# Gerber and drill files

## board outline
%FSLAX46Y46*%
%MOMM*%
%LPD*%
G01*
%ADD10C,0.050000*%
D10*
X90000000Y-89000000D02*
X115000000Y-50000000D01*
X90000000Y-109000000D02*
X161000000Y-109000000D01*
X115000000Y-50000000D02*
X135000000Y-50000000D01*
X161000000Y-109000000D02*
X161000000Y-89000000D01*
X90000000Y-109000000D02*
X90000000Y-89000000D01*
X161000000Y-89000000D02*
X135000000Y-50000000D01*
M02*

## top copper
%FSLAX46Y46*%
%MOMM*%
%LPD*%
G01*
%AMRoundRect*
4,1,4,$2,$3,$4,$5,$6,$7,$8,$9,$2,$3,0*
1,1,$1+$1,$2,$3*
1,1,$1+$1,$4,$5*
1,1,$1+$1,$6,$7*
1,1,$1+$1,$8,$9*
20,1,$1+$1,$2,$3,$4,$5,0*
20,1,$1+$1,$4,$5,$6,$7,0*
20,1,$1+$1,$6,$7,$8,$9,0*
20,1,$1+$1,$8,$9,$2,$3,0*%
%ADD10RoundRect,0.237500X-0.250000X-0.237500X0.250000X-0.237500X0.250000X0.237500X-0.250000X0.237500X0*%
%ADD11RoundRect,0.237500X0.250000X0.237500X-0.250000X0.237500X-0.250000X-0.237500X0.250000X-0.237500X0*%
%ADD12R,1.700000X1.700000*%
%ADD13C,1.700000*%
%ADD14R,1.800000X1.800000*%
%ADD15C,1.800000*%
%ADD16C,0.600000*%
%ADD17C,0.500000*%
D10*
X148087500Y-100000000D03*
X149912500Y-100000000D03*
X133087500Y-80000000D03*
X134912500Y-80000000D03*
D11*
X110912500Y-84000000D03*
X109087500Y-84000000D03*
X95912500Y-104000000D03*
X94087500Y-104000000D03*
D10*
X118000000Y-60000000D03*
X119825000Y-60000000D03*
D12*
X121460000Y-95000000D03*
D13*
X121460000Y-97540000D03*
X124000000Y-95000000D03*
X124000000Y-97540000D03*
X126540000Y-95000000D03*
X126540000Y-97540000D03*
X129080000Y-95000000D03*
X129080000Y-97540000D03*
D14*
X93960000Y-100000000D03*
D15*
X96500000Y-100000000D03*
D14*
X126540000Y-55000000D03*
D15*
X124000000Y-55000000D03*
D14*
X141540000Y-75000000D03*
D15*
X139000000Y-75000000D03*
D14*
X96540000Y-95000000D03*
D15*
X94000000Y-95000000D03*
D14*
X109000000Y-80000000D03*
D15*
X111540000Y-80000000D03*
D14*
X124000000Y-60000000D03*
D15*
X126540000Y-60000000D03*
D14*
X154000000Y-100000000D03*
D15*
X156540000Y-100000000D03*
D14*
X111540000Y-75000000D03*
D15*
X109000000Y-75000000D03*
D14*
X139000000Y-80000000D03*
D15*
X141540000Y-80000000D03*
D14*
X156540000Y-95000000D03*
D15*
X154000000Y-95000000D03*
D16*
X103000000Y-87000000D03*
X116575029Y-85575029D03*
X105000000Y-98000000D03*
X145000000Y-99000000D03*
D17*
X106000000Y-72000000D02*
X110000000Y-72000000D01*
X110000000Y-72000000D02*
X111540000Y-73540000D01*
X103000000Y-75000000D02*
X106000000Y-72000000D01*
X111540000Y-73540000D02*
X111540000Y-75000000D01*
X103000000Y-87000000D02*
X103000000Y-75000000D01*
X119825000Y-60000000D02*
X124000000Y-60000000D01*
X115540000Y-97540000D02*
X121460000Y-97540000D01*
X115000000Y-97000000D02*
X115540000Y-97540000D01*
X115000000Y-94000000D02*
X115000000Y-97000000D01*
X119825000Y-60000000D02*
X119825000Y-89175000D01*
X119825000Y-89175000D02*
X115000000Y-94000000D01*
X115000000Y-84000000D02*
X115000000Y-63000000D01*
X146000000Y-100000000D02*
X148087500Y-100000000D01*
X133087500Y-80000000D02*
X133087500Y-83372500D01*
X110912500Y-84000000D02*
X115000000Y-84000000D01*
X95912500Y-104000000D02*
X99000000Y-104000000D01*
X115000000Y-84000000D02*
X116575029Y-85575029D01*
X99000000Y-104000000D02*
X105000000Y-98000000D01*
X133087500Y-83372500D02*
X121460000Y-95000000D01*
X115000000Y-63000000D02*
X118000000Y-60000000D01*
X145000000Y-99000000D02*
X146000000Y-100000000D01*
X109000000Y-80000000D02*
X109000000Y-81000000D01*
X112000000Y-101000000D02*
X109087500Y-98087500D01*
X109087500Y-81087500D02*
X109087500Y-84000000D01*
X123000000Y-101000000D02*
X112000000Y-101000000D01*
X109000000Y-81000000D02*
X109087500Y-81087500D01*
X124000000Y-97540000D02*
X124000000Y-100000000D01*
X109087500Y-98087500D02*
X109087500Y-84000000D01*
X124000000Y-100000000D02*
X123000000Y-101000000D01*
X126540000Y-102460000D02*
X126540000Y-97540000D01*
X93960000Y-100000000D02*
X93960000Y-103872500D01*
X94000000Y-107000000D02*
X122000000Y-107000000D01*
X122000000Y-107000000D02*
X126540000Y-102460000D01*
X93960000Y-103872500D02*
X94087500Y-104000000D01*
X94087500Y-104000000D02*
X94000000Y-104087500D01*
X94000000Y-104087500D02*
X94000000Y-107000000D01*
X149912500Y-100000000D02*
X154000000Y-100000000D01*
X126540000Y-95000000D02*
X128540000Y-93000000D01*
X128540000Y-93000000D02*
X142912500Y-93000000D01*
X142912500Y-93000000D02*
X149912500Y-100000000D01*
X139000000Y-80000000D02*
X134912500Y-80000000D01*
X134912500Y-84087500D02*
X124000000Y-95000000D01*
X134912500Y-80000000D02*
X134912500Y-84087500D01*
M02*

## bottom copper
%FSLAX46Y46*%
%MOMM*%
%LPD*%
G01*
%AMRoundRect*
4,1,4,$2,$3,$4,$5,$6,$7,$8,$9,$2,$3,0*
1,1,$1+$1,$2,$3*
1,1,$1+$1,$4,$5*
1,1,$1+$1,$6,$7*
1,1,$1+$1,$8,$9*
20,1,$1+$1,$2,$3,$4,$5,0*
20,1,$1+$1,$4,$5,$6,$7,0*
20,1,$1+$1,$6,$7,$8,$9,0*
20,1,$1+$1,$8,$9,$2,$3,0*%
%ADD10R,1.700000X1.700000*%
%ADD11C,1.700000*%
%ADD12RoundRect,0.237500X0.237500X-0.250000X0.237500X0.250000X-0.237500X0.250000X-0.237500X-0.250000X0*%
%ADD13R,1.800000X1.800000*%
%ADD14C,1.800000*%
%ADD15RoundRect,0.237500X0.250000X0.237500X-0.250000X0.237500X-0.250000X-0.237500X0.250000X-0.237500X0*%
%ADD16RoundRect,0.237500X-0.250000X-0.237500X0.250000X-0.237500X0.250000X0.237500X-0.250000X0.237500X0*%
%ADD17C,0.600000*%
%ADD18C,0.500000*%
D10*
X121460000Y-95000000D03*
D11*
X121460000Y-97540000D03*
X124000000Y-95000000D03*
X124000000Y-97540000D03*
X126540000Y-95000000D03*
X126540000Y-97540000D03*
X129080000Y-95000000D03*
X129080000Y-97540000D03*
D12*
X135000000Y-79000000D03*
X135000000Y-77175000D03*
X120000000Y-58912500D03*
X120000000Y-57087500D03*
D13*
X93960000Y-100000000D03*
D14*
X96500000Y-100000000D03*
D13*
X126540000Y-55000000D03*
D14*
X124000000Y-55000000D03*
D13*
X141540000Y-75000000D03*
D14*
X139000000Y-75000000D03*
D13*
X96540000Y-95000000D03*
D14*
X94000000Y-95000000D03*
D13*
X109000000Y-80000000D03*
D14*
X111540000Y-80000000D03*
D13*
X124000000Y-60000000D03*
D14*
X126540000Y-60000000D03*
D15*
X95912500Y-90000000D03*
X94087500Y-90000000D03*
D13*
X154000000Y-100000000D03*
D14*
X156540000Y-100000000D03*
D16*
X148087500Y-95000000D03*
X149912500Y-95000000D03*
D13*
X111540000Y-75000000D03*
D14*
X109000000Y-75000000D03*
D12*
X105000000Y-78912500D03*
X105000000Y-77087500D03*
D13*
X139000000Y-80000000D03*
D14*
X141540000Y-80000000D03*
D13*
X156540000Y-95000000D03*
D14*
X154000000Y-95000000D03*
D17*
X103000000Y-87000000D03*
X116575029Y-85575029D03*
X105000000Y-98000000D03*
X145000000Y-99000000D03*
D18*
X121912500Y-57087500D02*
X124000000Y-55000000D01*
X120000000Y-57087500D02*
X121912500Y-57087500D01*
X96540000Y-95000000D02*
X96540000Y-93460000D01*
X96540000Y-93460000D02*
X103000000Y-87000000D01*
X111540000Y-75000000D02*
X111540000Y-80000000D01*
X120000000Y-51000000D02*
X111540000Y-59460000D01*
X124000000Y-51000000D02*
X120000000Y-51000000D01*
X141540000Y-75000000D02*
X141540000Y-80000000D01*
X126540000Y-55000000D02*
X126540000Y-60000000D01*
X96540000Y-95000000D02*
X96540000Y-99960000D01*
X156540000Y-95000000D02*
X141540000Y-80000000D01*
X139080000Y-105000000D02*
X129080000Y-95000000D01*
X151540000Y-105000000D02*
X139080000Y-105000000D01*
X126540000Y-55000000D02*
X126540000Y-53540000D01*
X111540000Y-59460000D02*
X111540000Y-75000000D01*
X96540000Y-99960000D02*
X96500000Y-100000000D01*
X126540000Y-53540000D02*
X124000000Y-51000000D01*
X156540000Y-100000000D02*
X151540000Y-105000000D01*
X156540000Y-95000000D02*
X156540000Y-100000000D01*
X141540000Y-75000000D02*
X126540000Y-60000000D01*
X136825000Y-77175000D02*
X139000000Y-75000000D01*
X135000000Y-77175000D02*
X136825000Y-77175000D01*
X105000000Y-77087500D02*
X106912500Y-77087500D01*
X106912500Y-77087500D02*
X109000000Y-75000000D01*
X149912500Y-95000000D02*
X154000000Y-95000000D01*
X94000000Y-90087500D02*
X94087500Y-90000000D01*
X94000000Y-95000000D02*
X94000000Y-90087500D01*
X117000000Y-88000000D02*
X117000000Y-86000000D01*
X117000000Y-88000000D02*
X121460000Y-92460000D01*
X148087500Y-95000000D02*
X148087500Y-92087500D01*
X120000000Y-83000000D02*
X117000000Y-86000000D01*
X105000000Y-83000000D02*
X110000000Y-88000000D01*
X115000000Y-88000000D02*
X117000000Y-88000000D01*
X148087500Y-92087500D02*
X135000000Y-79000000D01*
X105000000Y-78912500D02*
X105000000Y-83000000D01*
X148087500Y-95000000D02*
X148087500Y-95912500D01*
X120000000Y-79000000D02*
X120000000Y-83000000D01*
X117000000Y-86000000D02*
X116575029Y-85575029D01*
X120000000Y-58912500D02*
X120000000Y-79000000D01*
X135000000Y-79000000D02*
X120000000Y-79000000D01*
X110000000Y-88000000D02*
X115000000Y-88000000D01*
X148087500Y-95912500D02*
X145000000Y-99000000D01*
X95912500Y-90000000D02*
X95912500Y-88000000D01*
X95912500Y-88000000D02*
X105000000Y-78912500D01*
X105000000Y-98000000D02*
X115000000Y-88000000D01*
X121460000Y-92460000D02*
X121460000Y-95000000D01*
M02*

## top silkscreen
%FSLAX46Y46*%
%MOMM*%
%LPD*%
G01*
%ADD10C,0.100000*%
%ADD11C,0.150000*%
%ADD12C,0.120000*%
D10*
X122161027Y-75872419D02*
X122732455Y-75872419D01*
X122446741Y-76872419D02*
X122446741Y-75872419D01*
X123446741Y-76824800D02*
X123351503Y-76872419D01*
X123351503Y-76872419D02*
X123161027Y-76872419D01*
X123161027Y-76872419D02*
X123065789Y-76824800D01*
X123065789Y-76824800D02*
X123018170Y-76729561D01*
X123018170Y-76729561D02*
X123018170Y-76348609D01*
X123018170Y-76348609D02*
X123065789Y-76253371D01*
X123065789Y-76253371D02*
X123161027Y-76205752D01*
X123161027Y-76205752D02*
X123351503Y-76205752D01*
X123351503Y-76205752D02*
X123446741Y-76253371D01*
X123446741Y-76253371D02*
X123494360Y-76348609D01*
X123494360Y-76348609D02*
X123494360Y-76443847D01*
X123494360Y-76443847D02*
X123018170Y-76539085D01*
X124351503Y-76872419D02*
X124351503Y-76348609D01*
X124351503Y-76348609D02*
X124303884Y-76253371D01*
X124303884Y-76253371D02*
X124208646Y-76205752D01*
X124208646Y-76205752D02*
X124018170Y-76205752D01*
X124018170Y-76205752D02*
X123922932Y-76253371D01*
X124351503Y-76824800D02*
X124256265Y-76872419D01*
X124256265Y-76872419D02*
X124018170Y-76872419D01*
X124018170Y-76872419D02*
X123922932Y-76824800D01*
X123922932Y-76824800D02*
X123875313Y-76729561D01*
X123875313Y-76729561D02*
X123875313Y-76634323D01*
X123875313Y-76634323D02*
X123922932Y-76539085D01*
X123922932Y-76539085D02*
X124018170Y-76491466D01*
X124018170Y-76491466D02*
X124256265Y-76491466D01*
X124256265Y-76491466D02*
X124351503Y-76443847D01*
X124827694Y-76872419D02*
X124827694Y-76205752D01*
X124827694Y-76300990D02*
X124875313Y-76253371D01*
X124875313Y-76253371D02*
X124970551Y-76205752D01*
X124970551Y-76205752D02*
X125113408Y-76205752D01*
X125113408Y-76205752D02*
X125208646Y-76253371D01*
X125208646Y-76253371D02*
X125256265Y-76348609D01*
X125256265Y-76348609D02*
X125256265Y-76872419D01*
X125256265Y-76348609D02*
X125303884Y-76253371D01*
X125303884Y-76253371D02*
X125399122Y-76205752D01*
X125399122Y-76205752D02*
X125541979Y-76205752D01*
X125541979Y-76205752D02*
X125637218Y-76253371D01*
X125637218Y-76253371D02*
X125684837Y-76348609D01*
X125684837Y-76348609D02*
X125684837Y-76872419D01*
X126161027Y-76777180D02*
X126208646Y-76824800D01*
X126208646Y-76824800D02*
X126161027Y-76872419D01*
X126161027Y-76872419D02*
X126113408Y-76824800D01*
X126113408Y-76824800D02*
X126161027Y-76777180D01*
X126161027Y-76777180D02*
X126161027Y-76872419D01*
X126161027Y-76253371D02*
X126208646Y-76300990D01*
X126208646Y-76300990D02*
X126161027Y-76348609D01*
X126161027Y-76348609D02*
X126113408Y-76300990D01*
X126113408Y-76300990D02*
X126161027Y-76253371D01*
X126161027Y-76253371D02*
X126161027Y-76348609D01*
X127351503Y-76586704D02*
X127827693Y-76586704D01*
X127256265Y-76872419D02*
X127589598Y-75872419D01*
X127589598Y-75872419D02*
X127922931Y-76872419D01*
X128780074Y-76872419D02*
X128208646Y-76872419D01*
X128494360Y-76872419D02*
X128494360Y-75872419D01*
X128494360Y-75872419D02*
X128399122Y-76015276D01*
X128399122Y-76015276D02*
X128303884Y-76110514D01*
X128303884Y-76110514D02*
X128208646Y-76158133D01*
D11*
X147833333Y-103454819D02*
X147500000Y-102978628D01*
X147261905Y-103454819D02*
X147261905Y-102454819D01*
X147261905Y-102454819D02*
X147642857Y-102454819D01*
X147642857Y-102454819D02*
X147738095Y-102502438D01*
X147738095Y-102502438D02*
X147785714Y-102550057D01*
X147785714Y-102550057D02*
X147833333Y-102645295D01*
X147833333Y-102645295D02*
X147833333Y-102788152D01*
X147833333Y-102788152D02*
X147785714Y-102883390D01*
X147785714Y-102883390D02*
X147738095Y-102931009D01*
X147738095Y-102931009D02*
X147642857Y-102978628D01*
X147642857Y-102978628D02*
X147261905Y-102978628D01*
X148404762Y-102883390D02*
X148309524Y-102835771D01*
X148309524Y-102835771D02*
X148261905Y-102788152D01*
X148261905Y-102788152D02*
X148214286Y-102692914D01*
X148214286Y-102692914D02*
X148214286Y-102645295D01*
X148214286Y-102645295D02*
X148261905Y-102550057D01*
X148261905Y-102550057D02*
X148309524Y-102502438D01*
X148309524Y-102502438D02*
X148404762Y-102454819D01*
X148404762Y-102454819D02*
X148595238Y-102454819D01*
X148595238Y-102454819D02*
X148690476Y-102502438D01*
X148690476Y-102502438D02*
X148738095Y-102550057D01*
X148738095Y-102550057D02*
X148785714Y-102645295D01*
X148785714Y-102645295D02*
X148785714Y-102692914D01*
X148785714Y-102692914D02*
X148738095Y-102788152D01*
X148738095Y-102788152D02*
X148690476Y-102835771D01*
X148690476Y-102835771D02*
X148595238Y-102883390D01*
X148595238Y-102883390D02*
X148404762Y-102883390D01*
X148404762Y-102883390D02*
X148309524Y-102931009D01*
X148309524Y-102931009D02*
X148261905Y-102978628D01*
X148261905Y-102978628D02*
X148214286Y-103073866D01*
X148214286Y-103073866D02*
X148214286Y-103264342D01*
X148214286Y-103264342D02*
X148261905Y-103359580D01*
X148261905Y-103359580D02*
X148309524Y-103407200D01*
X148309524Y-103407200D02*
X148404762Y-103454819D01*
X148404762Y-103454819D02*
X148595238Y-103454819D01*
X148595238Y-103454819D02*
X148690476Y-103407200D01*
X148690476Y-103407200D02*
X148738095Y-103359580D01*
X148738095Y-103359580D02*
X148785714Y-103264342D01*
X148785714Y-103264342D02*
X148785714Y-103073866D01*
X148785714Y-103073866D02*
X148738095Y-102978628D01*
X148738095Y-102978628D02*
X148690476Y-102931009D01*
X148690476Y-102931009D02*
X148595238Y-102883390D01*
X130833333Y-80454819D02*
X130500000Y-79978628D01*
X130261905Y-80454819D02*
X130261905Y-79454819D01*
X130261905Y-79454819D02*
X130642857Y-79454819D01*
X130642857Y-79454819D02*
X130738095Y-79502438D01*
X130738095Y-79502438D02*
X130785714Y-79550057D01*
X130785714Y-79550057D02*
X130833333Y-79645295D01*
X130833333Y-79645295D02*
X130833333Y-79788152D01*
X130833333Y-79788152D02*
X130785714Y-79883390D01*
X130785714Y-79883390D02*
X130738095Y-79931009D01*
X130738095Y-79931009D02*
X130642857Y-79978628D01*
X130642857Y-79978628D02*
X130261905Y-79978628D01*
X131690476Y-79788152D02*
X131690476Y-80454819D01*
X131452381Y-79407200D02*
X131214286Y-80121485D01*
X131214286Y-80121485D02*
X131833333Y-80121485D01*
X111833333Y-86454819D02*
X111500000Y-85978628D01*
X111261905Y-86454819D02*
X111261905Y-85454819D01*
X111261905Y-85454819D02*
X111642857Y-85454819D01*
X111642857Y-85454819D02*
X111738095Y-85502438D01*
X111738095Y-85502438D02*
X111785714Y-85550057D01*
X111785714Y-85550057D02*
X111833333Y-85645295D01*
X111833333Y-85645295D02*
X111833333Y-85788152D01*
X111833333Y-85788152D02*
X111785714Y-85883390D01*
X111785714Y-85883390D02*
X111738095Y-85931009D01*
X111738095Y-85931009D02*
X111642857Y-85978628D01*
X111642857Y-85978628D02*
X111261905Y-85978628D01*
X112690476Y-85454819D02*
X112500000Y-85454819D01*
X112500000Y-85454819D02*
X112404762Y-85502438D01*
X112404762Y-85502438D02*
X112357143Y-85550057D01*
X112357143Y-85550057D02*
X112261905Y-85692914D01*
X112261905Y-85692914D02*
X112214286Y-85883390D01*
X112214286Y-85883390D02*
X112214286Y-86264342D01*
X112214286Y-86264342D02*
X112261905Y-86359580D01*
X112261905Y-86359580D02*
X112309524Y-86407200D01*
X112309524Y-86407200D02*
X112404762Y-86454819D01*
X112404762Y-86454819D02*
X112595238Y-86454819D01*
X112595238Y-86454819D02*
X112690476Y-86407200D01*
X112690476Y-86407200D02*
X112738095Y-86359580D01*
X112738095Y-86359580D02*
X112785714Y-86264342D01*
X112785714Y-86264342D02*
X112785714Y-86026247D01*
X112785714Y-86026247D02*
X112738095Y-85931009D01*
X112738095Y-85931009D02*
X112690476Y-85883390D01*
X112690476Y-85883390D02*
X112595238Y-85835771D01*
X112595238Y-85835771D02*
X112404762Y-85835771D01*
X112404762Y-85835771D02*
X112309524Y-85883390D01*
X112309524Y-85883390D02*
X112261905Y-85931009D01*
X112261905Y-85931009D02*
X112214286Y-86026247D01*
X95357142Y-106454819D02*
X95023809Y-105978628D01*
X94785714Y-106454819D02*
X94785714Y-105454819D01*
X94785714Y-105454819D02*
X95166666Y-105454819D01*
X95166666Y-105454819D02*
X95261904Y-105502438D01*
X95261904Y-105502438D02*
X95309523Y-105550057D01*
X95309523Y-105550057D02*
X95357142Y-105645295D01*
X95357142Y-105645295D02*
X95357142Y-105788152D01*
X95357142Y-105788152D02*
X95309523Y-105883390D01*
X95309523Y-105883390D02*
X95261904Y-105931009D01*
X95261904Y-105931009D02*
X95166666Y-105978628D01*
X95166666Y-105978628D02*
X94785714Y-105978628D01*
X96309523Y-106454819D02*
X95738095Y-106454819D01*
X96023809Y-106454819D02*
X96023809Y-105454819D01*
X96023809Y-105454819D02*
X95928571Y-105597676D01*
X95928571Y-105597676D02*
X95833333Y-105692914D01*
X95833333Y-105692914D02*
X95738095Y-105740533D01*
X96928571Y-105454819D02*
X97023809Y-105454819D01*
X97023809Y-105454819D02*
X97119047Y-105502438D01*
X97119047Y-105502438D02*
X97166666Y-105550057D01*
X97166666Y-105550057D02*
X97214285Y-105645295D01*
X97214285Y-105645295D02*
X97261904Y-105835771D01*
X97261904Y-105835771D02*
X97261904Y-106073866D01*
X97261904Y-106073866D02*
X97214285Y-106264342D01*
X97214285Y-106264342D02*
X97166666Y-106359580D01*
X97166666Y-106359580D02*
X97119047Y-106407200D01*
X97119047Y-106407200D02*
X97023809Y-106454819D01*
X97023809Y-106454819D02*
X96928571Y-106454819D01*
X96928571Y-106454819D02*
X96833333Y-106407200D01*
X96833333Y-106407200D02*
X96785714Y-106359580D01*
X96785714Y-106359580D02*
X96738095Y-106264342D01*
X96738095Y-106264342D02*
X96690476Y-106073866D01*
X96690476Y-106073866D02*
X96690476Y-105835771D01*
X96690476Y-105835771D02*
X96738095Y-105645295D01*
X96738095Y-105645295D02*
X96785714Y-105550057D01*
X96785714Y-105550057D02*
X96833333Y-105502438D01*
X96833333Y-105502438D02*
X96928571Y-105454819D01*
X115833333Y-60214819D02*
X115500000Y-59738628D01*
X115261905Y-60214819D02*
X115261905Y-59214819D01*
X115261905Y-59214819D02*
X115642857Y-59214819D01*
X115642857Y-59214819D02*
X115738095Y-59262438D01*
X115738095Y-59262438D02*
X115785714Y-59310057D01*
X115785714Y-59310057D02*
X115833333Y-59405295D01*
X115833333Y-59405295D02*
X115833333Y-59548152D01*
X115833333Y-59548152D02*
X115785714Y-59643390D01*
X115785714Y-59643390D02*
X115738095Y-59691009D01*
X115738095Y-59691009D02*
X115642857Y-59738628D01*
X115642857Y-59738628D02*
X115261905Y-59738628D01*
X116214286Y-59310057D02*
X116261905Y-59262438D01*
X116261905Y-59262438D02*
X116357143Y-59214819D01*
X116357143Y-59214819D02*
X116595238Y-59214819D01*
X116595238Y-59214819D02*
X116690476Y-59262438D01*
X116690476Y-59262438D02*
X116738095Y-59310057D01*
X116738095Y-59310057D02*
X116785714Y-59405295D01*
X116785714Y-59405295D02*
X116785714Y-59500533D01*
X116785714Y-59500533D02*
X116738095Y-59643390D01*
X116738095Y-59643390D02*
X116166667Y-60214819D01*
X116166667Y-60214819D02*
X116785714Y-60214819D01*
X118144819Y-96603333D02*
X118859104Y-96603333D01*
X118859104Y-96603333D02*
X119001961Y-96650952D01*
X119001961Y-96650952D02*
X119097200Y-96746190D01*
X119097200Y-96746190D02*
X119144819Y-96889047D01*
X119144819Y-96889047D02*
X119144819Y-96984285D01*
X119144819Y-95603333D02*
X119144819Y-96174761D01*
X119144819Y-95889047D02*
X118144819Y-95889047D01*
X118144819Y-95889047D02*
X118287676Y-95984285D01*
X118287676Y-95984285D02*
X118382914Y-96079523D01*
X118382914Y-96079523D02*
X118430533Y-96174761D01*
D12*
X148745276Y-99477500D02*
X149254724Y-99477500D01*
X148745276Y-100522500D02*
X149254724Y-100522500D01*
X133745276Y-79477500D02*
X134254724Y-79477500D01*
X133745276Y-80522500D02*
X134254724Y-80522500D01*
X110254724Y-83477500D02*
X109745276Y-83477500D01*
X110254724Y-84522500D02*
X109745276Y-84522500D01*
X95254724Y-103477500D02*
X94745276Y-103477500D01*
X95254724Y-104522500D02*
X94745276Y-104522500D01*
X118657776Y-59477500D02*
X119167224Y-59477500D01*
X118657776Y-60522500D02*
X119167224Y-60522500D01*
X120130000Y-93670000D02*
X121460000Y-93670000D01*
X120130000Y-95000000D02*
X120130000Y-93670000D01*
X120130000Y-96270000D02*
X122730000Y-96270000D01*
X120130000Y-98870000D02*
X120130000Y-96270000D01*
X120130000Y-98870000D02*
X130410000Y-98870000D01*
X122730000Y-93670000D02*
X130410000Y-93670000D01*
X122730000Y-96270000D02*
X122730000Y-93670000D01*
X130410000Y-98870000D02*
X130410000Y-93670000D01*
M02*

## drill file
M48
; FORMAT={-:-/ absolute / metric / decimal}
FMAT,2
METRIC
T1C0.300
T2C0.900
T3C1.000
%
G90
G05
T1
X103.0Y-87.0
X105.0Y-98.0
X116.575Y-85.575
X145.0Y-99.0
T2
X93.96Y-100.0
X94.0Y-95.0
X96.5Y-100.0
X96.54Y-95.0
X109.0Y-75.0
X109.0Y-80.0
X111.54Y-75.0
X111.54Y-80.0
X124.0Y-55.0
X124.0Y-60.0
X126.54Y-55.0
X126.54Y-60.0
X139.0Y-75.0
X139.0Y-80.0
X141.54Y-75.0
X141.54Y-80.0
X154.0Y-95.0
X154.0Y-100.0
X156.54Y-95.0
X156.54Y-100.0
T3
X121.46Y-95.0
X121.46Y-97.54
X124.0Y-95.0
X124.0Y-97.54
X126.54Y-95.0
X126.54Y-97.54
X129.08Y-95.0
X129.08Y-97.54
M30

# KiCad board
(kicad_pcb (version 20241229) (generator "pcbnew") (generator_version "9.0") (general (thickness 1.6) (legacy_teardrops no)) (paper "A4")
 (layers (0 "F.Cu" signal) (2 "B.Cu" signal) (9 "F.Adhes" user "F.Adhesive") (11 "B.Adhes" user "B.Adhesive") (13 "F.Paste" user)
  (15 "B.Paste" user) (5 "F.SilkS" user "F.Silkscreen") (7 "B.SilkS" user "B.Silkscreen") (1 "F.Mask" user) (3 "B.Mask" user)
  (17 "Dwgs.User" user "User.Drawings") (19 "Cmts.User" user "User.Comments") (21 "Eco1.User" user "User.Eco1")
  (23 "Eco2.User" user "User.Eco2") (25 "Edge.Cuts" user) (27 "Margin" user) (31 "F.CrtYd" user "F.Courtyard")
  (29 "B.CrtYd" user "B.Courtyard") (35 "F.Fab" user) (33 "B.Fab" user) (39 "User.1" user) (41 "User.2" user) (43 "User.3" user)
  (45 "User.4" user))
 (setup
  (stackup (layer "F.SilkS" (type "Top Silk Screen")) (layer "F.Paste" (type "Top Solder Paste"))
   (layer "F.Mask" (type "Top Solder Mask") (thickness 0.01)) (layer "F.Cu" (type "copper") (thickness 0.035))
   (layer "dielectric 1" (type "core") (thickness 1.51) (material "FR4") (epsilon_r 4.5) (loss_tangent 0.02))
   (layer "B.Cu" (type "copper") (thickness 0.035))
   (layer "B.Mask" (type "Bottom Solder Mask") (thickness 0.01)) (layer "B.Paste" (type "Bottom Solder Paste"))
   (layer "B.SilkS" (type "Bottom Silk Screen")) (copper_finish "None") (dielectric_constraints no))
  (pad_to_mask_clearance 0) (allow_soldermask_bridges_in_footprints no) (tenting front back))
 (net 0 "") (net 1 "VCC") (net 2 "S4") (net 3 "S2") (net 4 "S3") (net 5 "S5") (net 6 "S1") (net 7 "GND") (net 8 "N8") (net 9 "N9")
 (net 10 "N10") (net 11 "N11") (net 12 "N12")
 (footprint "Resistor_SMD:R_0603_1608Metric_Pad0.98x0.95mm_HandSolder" (layer "F.Cu") (at 149 100)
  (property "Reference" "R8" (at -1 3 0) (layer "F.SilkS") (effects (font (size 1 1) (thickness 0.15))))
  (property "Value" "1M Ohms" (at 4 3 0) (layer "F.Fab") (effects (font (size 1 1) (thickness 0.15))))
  (fp_line (start -0.254724 -0.5225) (end 0.254724 -0.5225) (stroke (width 0.12) (type solid)) (layer "F.SilkS"))
  (fp_line (start -0.254724 0.5225) (end 0.254724 0.5225) (stroke (width 0.12) (type solid)) (layer "F.SilkS"))
  (pad "1" smd roundrect (at -0.9125 0) (size 0.975 0.95) (layers "F.Cu" "F.Mask" "F.Paste") (roundrect_rratio 0.25) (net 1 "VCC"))
  (pad "2" smd roundrect (at 0.9125 0) (size 0.975 0.95) (layers "F.Cu" "F.Mask" "F.Paste") (roundrect_rratio 0.25) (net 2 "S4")))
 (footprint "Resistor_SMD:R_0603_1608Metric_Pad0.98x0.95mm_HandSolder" (layer "F.Cu") (at 134 80)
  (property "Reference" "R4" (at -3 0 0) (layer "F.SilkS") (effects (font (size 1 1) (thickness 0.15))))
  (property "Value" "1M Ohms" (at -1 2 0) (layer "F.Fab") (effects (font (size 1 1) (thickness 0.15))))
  (fp_line (start -0.254724 -0.5225) (end 0.254724 -0.5225) (stroke (width 0.12) (type solid)) (layer "F.SilkS"))
  (fp_line (start -0.254724 0.5225) (end 0.254724 0.5225) (stroke (width 0.12) (type solid)) (layer "F.SilkS"))
  (pad "1" smd roundrect (at -0.9125 0) (size 0.975 0.95) (layers "F.Cu" "F.Mask" "F.Paste") (roundrect_rratio 0.25) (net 1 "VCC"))
  (pad "2" smd roundrect (at 0.9125 0) (size 0.975 0.95) (layers "F.Cu" "F.Mask" "F.Paste") (roundrect_rratio 0.25) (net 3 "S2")))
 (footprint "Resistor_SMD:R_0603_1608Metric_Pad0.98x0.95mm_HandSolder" (layer "F.Cu") (at 110 84 180)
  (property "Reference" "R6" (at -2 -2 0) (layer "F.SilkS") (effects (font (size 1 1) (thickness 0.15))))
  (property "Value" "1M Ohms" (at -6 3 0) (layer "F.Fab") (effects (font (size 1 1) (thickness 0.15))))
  (fp_line (start -0.254724 0.5225) (end 0.254724 0.5225) (stroke (width 0.12) (type solid)) (layer "F.SilkS"))
  (fp_line (start -0.254724 -0.5225) (end 0.254724 -0.5225) (stroke (width 0.12) (type solid)) (layer "F.SilkS"))
  (pad "1" smd roundrect (at -0.9125 0 180) (size 0.975 0.95) (layers "F.Cu" "F.Mask" "F.Paste") (roundrect_rratio 0.25) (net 1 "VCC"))
  (pad "2" smd roundrect (at 0.9125 0 180) (size 0.975 0.95) (layers "F.Cu" "F.Mask" "F.Paste") (roundrect_rratio 0.25) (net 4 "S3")))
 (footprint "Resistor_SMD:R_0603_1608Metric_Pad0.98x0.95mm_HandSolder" (layer "F.Cu") (at 95 104 180)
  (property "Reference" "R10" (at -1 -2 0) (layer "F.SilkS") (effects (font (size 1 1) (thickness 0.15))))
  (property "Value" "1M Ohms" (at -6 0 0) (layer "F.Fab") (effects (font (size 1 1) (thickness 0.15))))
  (fp_line (start -0.254724 0.5225) (end 0.254724 0.5225) (stroke (width 0.12) (type solid)) (layer "F.SilkS"))
  (fp_line (start -0.254724 -0.5225) (end 0.254724 -0.5225) (stroke (width 0.12) (type solid)) (layer "F.SilkS"))
  (pad "1" smd roundrect (at -0.9125 0 180) (size 0.975 0.95) (layers "F.Cu" "F.Mask" "F.Paste") (roundrect_rratio 0.25) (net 1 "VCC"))
  (pad "2" smd roundrect (at 0.9125 0 180) (size 0.975 0.95) (layers "F.Cu" "F.Mask" "F.Paste") (roundrect_rratio 0.25) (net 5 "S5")))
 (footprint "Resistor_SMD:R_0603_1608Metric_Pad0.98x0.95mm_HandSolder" (layer "F.Cu") (at 118.9125 60)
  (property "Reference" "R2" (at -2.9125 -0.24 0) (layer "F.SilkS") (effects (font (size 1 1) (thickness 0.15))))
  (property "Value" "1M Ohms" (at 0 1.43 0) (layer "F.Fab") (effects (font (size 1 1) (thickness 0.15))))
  (fp_line (start -0.254724 -0.5225) (end 0.254724 -0.5225) (stroke (width 0.12) (type solid)) (layer "F.SilkS"))
  (fp_line (start -0.254724 0.5225) (end 0.254724 0.5225) (stroke (width 0.12) (type solid)) (layer "F.SilkS"))
  (pad "1" smd roundrect (at -0.9125 0) (size 0.975 0.95) (layers "F.Cu" "F.Mask" "F.Paste") (roundrect_rratio 0.25) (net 1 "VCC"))
  (pad "2" smd roundrect (at 0.9125 0) (size 0.975 0.95) (layers "F.Cu" "F.Mask" "F.Paste") (roundrect_rratio 0.25) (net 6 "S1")))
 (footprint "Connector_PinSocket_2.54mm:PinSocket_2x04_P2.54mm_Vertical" (layer "F.Cu") (at 121.46 95 90)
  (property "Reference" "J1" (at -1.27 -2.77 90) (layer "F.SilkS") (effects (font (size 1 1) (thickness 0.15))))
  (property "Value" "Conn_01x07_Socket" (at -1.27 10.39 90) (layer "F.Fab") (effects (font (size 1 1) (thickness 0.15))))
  (fp_line (start 1.33 -1.33) (end 1.33 0) (stroke (width 0.12) (type solid)) (layer "F.SilkS"))
  (fp_line (start 0 -1.33) (end 1.33 -1.33) (stroke (width 0.12) (type solid)) (layer "F.SilkS"))
  (fp_line (start -1.27 -1.33) (end -1.27 1.27) (stroke (width 0.12) (type solid)) (layer "F.SilkS"))
  (fp_line (start -3.87 -1.33) (end -1.27 -1.33) (stroke (width 0.12) (type solid)) (layer "F.SilkS"))
  (fp_line (start -3.87 -1.33) (end -3.87 8.95) (stroke (width 0.12) (type solid)) (layer "F.SilkS"))
  (fp_line (start 1.33 1.27) (end 1.33 8.95) (stroke (width 0.12) (type solid)) (layer "F.SilkS"))
  (fp_line (start -1.27 1.27) (end 1.33 1.27) (stroke (width 0.12) (type solid)) (layer "F.SilkS"))
  (fp_line (start -3.87 8.95) (end 1.33 8.95) (stroke (width 0.12) (type solid)) (layer "F.SilkS"))
  (pad "1" thru_hole rect (at 0 0 90) (size 1.7 1.7) (drill 1) (layers "*.Cu" "*.Mask") (remove_unused_layers no) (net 1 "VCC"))
  (pad "2" thru_hole circle (at -2.54 0 90) (size 1.7 1.7) (drill 1) (layers "*.Cu" "*.Mask") (remove_unused_layers no) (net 6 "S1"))
  (pad "3" thru_hole circle (at 0 2.54 90) (size 1.7 1.7) (drill 1) (layers "*.Cu" "*.Mask") (remove_unused_layers no) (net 3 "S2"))
  (pad "4" thru_hole circle (at -2.54 2.54 90) (size 1.7 1.7) (drill 1) (layers "*.Cu" "*.Mask") (remove_unused_layers no) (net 4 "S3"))
  (pad "5" thru_hole circle (at 0 5.08 90) (size 1.7 1.7) (drill 1) (layers "*.Cu" "*.Mask") (remove_unused_layers no) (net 2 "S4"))
  (pad "6" thru_hole circle (at -2.54 5.08 90) (size 1.7 1.7) (drill 1) (layers "*.Cu" "*.Mask") (remove_unused_layers no) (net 5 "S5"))
  (pad "7" thru_hole circle (at 0 7.62 90) (size 1.7 1.7) (drill 1) (layers "*.Cu" "*.Mask") (remove_unused_layers no) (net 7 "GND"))
  (pad "8" thru_hole circle (at -2.54 7.62 90) (size 1.7 1.7) (drill 1) (layers "*.Cu" "*.Mask") (remove_unused_layers no)))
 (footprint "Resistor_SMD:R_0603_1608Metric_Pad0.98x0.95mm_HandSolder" (layer "B.Cu") (at 135 78.0875 90)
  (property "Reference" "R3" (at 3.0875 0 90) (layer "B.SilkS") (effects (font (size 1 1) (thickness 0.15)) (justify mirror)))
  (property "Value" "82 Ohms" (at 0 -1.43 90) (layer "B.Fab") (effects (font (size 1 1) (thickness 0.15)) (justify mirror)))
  (pad "1" smd roundrect (at -0.9125 0 90) (size 0.975 0.95) (layers "B.Cu" "B.Mask" "B.Paste") (roundrect_rratio 0.25) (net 1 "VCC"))
  (pad "2" smd roundrect (at 0.9125 0 90) (size 0.975 0.95) (layers "B.Cu" "B.Mask" "B.Paste") (roundrect_rratio 0.25) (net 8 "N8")))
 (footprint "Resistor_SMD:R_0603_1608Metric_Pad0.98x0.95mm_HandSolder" (layer "B.Cu") (at 120 58 90)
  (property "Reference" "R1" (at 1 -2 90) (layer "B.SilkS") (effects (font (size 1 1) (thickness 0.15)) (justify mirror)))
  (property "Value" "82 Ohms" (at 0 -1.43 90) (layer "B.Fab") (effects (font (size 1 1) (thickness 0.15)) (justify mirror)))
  (pad "1" smd roundrect (at -0.9125 0 90) (size 0.975 0.95) (layers "B.Cu" "B.Mask" "B.Paste") (roundrect_rratio 0.25) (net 1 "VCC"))
  (pad "2" smd roundrect (at 0.9125 0 90) (size 0.975 0.95) (layers "B.Cu" "B.Mask" "B.Paste") (roundrect_rratio 0.25) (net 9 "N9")))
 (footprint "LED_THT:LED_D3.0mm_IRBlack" (layer "B.Cu") (at 93.96 100)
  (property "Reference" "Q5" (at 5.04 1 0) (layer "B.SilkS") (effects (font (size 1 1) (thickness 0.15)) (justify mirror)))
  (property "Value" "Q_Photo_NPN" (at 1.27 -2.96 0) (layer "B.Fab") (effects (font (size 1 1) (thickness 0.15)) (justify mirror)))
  (pad "1" thru_hole rect (at 0 0) (size 1.8 1.8) (drill 0.9) (layers "*.Cu" "*.Mask") (remove_unused_layers no) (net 5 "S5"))
  (pad "2" thru_hole circle (at 2.54 0) (size 1.8 1.8) (drill 0.9) (layers "*.Cu" "*.Mask") (remove_unused_layers no) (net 7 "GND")))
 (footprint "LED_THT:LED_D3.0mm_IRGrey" (layer "B.Cu") (at 126.54 55 180)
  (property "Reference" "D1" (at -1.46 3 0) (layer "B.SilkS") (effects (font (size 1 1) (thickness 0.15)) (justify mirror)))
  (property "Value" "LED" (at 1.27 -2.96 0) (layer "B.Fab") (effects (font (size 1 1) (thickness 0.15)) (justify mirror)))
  (pad "1" thru_hole rect (at 0 0 180) (size 1.8 1.8) (drill 0.9) (layers "*.Cu" "*.Mask") (remove_unused_layers no) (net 7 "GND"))
  (pad "2" thru_hole circle (at 2.54 0 180) (size 1.8 1.8) (drill 0.9) (layers "*.Cu" "*.Mask") (remove_unused_layers no) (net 9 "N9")))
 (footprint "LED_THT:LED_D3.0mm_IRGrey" (layer "B.Cu") (at 141.54 75 180)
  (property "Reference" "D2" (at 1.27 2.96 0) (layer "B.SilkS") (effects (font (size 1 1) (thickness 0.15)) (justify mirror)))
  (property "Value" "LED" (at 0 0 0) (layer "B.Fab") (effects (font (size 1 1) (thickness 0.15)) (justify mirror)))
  (pad "1" thru_hole rect (at 0 0 180) (size 1.8 1.8) (drill 0.9) (layers "*.Cu" "*.Mask") (remove_unused_layers no) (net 7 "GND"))
  (pad "2" thru_hole circle (at 2.54 0 180) (size 1.8 1.8) (drill 0.9) (layers "*.Cu" "*.Mask") (remove_unused_layers no) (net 8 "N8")))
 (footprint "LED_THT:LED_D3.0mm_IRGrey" (layer "B.Cu") (at 96.54 95 180)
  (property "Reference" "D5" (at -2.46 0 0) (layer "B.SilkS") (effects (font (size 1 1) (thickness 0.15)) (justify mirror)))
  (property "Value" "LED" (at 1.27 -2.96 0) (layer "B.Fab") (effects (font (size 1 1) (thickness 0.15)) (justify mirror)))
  (pad "1" thru_hole rect (at 0 0 180) (size 1.8 1.8) (drill 0.9) (layers "*.Cu" "*.Mask") (remove_unused_layers no) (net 7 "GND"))
  (pad "2" thru_hole circle (at 2.54 0 180) (size 1.8 1.8) (drill 0.9) (layers "*.Cu" "*.Mask") (remove_unused_layers no) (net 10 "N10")))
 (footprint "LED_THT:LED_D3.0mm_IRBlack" (layer "B.Cu") (at 109 80)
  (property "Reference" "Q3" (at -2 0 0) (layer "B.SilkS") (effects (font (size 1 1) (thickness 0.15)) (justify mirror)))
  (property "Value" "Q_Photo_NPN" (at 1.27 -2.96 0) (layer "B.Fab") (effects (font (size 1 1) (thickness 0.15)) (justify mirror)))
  (pad "1" thru_hole rect (at 0 0) (size 1.8 1.8) (drill 0.9) (layers "*.Cu" "*.Mask") (remove_unused_layers no) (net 4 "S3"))
  (pad "2" thru_hole circle (at 2.54 0) (size 1.8 1.8) (drill 0.9) (layers "*.Cu" "*.Mask") (remove_unused_layers no) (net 7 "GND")))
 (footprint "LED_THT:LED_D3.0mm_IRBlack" (layer "B.Cu") (at 124 60)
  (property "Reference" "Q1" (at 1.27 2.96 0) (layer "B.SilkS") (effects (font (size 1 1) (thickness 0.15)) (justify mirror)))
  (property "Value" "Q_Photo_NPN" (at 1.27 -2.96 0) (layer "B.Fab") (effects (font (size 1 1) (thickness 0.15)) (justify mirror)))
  (pad "1" thru_hole rect (at 0 0) (size 1.8 1.8) (drill 0.9) (layers "*.Cu" "*.Mask") (remove_unused_layers no) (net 6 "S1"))
  (pad "2" thru_hole circle (at 2.54 0) (size 1.8 1.8) (drill 0.9) (layers "*.Cu" "*.Mask") (remove_unused_layers no) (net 7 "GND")))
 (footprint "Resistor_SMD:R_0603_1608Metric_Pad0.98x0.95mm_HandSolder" (layer "B.Cu") (at 95 90 180)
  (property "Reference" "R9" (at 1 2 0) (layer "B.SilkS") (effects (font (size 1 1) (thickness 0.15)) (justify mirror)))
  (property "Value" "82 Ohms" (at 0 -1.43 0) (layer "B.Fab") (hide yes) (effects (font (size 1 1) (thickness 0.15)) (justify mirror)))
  (pad "1" smd roundrect (at -0.9125 0 180) (size 0.975 0.95) (layers "B.Cu" "B.Mask" "B.Paste") (roundrect_rratio 0.25) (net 1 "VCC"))
  (pad "2" smd roundrect (at 0.9125 0 180) (size 0.975 0.95) (layers "B.Cu" "B.Mask" "B.Paste") (roundrect_rratio 0.25) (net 10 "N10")))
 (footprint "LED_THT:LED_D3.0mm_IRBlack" (layer "B.Cu") (at 154 100)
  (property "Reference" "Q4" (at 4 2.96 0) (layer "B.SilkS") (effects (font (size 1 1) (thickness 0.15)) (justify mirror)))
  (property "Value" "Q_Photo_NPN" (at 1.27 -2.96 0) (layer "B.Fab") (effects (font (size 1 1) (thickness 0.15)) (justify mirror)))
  (pad "1" thru_hole rect (at 0 0) (size 1.8 1.8) (drill 0.9) (layers "*.Cu" "*.Mask") (remove_unused_layers no) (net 2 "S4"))
  (pad "2" thru_hole circle (at 2.54 0) (size 1.8 1.8) (drill 0.9) (layers "*.Cu" "*.Mask") (remove_unused_layers no) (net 7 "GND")))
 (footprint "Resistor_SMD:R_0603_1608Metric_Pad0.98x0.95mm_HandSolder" (layer "B.Cu") (at 149 95)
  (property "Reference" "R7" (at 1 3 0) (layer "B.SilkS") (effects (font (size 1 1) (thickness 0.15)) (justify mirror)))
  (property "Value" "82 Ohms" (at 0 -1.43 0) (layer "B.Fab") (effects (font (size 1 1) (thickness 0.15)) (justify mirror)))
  (pad "1" smd roundrect (at -0.9125 0) (size 0.975 0.95) (layers "B.Cu" "B.Mask" "B.Paste") (roundrect_rratio 0.25) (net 1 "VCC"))
  (pad "2" smd roundrect (at 0.9125 0) (size 0.975 0.95) (layers "B.Cu" "B.Mask" "B.Paste") (roundrect_rratio 0.25) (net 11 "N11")))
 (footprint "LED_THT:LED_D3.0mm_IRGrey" (layer "B.Cu") (at 111.54 75 180)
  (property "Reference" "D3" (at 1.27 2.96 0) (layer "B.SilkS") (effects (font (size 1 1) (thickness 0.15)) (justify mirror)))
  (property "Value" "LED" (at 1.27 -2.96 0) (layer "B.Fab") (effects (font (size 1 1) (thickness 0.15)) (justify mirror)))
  (pad "1" thru_hole rect (at 0 0 180) (size 1.8 1.8) (drill 0.9) (layers "*.Cu" "*.Mask") (remove_unused_layers no) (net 7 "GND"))
  (pad "2" thru_hole circle (at 2.54 0 180) (size 1.8 1.8) (drill 0.9) (layers "*.Cu" "*.Mask") (remove_unused_layers no) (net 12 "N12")))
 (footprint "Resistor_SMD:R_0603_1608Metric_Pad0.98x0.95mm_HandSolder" (layer "B.Cu") (at 105 78 90)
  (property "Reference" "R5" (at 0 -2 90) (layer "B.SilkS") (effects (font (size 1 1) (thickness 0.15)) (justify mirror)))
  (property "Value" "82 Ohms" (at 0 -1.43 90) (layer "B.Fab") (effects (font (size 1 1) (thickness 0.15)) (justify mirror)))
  (pad "1" smd roundrect (at -0.9125 0 90) (size 0.975 0.95) (layers "B.Cu" "B.Mask" "B.Paste") (roundrect_rratio 0.25) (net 1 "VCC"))
  (pad "2" smd roundrect (at 0.9125 0 90) (size 0.975 0.95) (layers "B.Cu" "B.Mask" "B.Paste") (roundrect_rratio 0.25) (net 12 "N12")))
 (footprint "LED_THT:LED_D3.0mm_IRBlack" (layer "B.Cu") (at 139 80)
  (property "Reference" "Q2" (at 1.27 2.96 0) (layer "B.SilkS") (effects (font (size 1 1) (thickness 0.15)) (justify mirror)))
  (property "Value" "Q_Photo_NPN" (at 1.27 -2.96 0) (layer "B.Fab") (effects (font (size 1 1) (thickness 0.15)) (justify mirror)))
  (pad "1" thru_hole rect (at 0 0) (size 1.8 1.8) (drill 0.9) (layers "*.Cu" "*.Mask") (remove_unused_layers no) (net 3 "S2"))
  (pad "2" thru_hole circle (at 2.54 0) (size 1.8 1.8) (drill 0.9) (layers "*.Cu" "*.Mask") (remove_unused_layers no) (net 7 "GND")))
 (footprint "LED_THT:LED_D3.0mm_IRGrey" (layer "B.Cu") (at 156.54 95 180)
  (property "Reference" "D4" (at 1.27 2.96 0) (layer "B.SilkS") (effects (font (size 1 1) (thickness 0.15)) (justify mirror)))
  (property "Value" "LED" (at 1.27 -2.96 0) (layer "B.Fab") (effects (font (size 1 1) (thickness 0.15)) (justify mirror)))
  (pad "1" thru_hole rect (at 0 0 180) (size 1.8 1.8) (drill 0.9) (layers "*.Cu" "*.Mask") (remove_unused_layers no) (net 7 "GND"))
  (pad "2" thru_hole circle (at 2.54 0 180) (size 1.8 1.8) (drill 0.9) (layers "*.Cu" "*.Mask") (remove_unused_layers no) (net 11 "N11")))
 (gr_line (start 90 89) (end 115 50) (stroke (width 0.05) (type default)) (layer "Edge.Cuts"))
 (gr_line (start 90 109) (end 161 109) (stroke (width 0.05) (type default)) (layer "Edge.Cuts"))
 (gr_line (start 115 50) (end 135 50) (stroke (width 0.05) (type default)) (layer "Edge.Cuts"))
 (gr_line (start 161 109) (end 161 89) (stroke (width 0.05) (type default)) (layer "Edge.Cuts"))
 (gr_line (start 90 109) (end 90 89) (stroke (width 0.05) (type default)) (layer "Edge.Cuts"))
 (gr_line (start 161 89) (end 135 50) (stroke (width 0.05) (type default)) (layer "Edge.Cuts"))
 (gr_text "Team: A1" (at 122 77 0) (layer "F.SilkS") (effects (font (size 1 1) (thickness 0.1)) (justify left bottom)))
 (segment (start 121.9125 57.0875) (end 124 55) (width 0.5) (layer "B.Cu") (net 9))
 (segment (start 120 57.0875) (end 121.9125 57.0875) (width 0.5) (layer "B.Cu") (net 9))
 (segment (start 106 72) (end 110 72) (width 0.5) (layer "F.Cu") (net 7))
 (segment (start 110 72) (end 111.54 73.54) (width 0.5) (layer "F.Cu") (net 7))
 (segment (start 103 75) (end 106 72) (width 0.5) (layer "F.Cu") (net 7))
 (segment (start 111.54 73.54) (end 111.54 75) (width 0.5) (layer "F.Cu") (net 7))
 (segment (start 103 87) (end 103 75) (width 0.5) (layer "F.Cu") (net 7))
 (via (at 103 87) (size 0.6) (drill 0.3) (layers "F.Cu" "B.Cu") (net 7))
 (segment (start 96.54 95) (end 96.54 93.46) (width 0.5) (layer "B.Cu") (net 7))
 (segment (start 96.54 93.46) (end 103 87) (width 0.5) (layer "B.Cu") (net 7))
 (segment (start 111.54 75) (end 111.54 80) (width 0.5) (layer "B.Cu") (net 7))
 (segment (start 120 51) (end 111.54 59.46) (width 0.5) (layer "B.Cu") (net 7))
 (segment (start 124 51) (end 120 51) (width 0.5) (layer "B.Cu") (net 7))
 (segment (start 141.54 75) (end 141.54 80) (width 0.5) (layer "B.Cu") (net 7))
 (segment (start 126.54 55) (end 126.54 60) (width 0.5) (layer "B.Cu") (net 7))
 (segment (start 96.54 95) (end 96.54 99.96) (width 0.5) (layer "B.Cu") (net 7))
 (segment (start 156.54 95) (end 141.54 80) (width 0.5) (layer "B.Cu") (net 7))
 (segment (start 139.08 105) (end 129.08 95) (width 0.5) (layer "B.Cu") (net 7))
 (segment (start 151.54 105) (end 139.08 105) (width 0.5) (layer "B.Cu") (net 7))
 (segment (start 126.54 55) (end 126.54 53.54) (width 0.5) (layer "B.Cu") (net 7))
 (segment (start 111.54 59.46) (end 111.54 75) (width 0.5) (layer "B.Cu") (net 7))
 (segment (start 96.54 99.96) (end 96.5 100) (width 0.5) (layer "B.Cu") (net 7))
 (segment (start 126.54 53.54) (end 124 51) (width 0.5) (layer "B.Cu") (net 7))
 (segment (start 156.54 100) (end 151.54 105) (width 0.5) (layer "B.Cu") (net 7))
 (segment (start 156.54 95) (end 156.54 100) (width 0.5) (layer "B.Cu") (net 7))
 (segment (start 141.54 75) (end 126.54 60) (width 0.5) (layer "B.Cu") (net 7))
 (segment (start 136.825 77.175) (end 139 75) (width 0.5) (layer "B.Cu") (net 8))
 (segment (start 135 77.175) (end 136.825 77.175) (width 0.5) (layer "B.Cu") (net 8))
 (segment (start 105 77.0875) (end 106.9125 77.0875) (width 0.5) (layer "B.Cu") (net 12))
 (segment (start 106.9125 77.0875) (end 109 75) (width 0.5) (layer "B.Cu") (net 12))
 (segment (start 149.9125 95) (end 154 95) (width 0.5) (layer "B.Cu") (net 11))
 (segment (start 94 90.0875) (end 94.0875 90) (width 0.5) (layer "B.Cu") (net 10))
 (segment (start 94 95) (end 94 90.0875) (width 0.5) (layer "B.Cu") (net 10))
 (segment (start 119.825 60) (end 124 60) (width 0.5) (layer "F.Cu") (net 6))
 (segment (start 115.54 97.54) (end 121.46 97.54) (width 0.5) (layer "F.Cu") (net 6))
 (segment (start 115 97) (end 115.54 97.54) (width 0.5) (layer "F.Cu") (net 6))
 (segment (start 115 94) (end 115 97) (width 0.5) (layer "F.Cu") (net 6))
 (segment (start 119.825 60) (end 119.825 89.175) (width 0.5) (layer "F.Cu") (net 6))
 (segment (start 119.825 89.175) (end 115 94) (width 0.5) (layer "F.Cu") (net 6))
 (segment (start 115 84) (end 115 63) (width 0.5) (layer "F.Cu") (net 1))
 (segment (start 146 100) (end 148.0875 100) (width 0.5) (layer "F.Cu") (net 1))
 (segment (start 133.0875 80) (end 133.0875 83.3725) (width 0.5) (layer "F.Cu") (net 1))
 (segment (start 110.9125 84) (end 115 84) (width 0.5) (layer "F.Cu") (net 1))
 (segment (start 95.9125 104) (end 99 104) (width 0.5) (layer "F.Cu") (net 1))
 (segment (start 115 84) (end 116.575029 85.575029) (width 0.5) (layer "F.Cu") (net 1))
 (segment (start 99 104) (end 105 98) (width 0.5) (layer "F.Cu") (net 1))
 (segment (start 133.0875 83.3725) (end 121.46 95) (width 0.5) (layer "F.Cu") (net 1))
 (segment (start 115 63) (end 118 60) (width 0.5) (layer "F.Cu") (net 1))
 (segment (start 145 99) (end 146 100) (width 0.5) (layer "F.Cu") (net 1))
 (via (at 116.575029 85.575029) (size 0.6) (drill 0.3) (layers "F.Cu" "B.Cu") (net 1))
 (via (at 105 98) (size 0.6) (drill 0.3) (layers "F.Cu" "B.Cu") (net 1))
 (via (at 145 99) (size 0.6) (drill 0.3) (layers "F.Cu" "B.Cu") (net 1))
 (segment (start 117 88) (end 117 86) (width 0.5) (layer "B.Cu") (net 1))
 (segment (start 117 88) (end 121.46 92.46) (width 0.5) (layer "B.Cu") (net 1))
 (segment (start 148.0875 95) (end 148.0875 92.0875) (width 0.5) (layer "B.Cu") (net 1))
 (segment (start 120 83) (end 117 86) (width 0.5) (layer "B.Cu") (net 1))
 (segment (start 105 83) (end 110 88) (width 0.5) (layer "B.Cu") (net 1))
 (segment (start 115 88) (end 117 88) (width 0.5) (layer "B.Cu") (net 1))
 (segment (start 148.0875 92.0875) (end 135 79) (width 0.5) (layer "B.Cu") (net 1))
 (segment (start 105 78.9125) (end 105 83) (width 0.5) (layer "B.Cu") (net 1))
 (segment (start 148.0875 95) (end 148.0875 95.9125) (width 0.5) (layer "B.Cu") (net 1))
 (segment (start 120 79) (end 120 83) (width 0.5) (layer "B.Cu") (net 1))
 (segment (start 117 86) (end 116.575029 85.575029) (width 0.5) (layer "B.Cu") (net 1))
 (segment (start 120 58.9125) (end 120 79) (width 0.5) (layer "B.Cu") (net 1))
 (segment (start 135 79) (end 120 79) (width 0.5) (layer "B.Cu") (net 1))
 (segment (start 110 88) (end 115 88) (width 0.5) (layer "B.Cu") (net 1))
 (segment (start 148.0875 95.9125) (end 145 99) (width 0.5) (layer "B.Cu") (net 1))
 (segment (start 95.9125 90) (end 95.9125 88) (width 0.5) (layer "B.Cu") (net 1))
 (segment (start 95.9125 88) (end 105 78.9125) (width 0.5) (layer "B.Cu") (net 1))
 (segment (start 105 98) (end 115 88) (width 0.5) (layer "B.Cu") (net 1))
 (segment (start 121.46 92.46) (end 121.46 95) (width 0.5) (layer "B.Cu") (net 1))
 (segment (start 109 80) (end 109 81) (width 0.5) (layer "F.Cu") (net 4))
 (segment (start 112 101) (end 109.0875 98.0875) (width 0.5) (layer "F.Cu") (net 4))
 (segment (start 109.0875 81.0875) (end 109.0875 84) (width 0.5) (layer "F.Cu") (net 4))
 (segment (start 123 101) (end 112 101) (width 0.5) (layer "F.Cu") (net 4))
 (segment (start 109 81) (end 109.0875 81.0875) (width 0.5) (layer "F.Cu") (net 4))
 (segment (start 124 97.54) (end 124 100) (width 0.5) (layer "F.Cu") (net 4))
 (segment (start 109.0875 98.0875) (end 109.0875 84) (width 0.5) (layer "F.Cu") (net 4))
 (segment (start 124 100) (end 123 101) (width 0.5) (layer "F.Cu") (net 4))
 (segment (start 126.54 102.46) (end 126.54 97.54) (width 0.5) (layer "F.Cu") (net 5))
 (segment (start 93.96 100) (end 93.96 103.8725) (width 0.5) (layer "F.Cu") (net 5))
 (segment (start 94 107) (end 122 107) (width 0.5) (layer "F.Cu") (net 5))
 (segment (start 122 107) (end 126.54 102.46) (width 0.5) (layer "F.Cu") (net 5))
 (segment (start 93.96 103.8725) (end 94.0875 104) (width 0.5) (layer "F.Cu") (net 5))
 (segment (start 94.0875 104) (end 94 104.0875) (width 0.5) (layer "F.Cu") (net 5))
 (segment (start 94 104.0875) (end 94 107) (width 0.5) (layer "F.Cu") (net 5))
 (segment (start 149.9125 100) (end 154 100) (width 0.5) (layer "F.Cu") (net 2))
 (segment (start 126.54 95) (end 128.54 93) (width 0.5) (layer "F.Cu") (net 2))
 (segment (start 128.54 93) (end 142.9125 93) (width 0.5) (layer "F.Cu") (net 2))
 (segment (start 142.9125 93) (end 149.9125 100) (width 0.5) (layer "F.Cu") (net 2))
 (segment (start 139 80) (end 134.9125 80) (width 0.5) (layer "F.Cu") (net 3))
 (segment (start 134.9125 84.0875) (end 124 95) (width 0.5) (layer "F.Cu") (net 3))
 (segment (start 134.9125 80) (end 134.9125 84.0875) (width 0.5) (layer "F.Cu") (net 3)))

